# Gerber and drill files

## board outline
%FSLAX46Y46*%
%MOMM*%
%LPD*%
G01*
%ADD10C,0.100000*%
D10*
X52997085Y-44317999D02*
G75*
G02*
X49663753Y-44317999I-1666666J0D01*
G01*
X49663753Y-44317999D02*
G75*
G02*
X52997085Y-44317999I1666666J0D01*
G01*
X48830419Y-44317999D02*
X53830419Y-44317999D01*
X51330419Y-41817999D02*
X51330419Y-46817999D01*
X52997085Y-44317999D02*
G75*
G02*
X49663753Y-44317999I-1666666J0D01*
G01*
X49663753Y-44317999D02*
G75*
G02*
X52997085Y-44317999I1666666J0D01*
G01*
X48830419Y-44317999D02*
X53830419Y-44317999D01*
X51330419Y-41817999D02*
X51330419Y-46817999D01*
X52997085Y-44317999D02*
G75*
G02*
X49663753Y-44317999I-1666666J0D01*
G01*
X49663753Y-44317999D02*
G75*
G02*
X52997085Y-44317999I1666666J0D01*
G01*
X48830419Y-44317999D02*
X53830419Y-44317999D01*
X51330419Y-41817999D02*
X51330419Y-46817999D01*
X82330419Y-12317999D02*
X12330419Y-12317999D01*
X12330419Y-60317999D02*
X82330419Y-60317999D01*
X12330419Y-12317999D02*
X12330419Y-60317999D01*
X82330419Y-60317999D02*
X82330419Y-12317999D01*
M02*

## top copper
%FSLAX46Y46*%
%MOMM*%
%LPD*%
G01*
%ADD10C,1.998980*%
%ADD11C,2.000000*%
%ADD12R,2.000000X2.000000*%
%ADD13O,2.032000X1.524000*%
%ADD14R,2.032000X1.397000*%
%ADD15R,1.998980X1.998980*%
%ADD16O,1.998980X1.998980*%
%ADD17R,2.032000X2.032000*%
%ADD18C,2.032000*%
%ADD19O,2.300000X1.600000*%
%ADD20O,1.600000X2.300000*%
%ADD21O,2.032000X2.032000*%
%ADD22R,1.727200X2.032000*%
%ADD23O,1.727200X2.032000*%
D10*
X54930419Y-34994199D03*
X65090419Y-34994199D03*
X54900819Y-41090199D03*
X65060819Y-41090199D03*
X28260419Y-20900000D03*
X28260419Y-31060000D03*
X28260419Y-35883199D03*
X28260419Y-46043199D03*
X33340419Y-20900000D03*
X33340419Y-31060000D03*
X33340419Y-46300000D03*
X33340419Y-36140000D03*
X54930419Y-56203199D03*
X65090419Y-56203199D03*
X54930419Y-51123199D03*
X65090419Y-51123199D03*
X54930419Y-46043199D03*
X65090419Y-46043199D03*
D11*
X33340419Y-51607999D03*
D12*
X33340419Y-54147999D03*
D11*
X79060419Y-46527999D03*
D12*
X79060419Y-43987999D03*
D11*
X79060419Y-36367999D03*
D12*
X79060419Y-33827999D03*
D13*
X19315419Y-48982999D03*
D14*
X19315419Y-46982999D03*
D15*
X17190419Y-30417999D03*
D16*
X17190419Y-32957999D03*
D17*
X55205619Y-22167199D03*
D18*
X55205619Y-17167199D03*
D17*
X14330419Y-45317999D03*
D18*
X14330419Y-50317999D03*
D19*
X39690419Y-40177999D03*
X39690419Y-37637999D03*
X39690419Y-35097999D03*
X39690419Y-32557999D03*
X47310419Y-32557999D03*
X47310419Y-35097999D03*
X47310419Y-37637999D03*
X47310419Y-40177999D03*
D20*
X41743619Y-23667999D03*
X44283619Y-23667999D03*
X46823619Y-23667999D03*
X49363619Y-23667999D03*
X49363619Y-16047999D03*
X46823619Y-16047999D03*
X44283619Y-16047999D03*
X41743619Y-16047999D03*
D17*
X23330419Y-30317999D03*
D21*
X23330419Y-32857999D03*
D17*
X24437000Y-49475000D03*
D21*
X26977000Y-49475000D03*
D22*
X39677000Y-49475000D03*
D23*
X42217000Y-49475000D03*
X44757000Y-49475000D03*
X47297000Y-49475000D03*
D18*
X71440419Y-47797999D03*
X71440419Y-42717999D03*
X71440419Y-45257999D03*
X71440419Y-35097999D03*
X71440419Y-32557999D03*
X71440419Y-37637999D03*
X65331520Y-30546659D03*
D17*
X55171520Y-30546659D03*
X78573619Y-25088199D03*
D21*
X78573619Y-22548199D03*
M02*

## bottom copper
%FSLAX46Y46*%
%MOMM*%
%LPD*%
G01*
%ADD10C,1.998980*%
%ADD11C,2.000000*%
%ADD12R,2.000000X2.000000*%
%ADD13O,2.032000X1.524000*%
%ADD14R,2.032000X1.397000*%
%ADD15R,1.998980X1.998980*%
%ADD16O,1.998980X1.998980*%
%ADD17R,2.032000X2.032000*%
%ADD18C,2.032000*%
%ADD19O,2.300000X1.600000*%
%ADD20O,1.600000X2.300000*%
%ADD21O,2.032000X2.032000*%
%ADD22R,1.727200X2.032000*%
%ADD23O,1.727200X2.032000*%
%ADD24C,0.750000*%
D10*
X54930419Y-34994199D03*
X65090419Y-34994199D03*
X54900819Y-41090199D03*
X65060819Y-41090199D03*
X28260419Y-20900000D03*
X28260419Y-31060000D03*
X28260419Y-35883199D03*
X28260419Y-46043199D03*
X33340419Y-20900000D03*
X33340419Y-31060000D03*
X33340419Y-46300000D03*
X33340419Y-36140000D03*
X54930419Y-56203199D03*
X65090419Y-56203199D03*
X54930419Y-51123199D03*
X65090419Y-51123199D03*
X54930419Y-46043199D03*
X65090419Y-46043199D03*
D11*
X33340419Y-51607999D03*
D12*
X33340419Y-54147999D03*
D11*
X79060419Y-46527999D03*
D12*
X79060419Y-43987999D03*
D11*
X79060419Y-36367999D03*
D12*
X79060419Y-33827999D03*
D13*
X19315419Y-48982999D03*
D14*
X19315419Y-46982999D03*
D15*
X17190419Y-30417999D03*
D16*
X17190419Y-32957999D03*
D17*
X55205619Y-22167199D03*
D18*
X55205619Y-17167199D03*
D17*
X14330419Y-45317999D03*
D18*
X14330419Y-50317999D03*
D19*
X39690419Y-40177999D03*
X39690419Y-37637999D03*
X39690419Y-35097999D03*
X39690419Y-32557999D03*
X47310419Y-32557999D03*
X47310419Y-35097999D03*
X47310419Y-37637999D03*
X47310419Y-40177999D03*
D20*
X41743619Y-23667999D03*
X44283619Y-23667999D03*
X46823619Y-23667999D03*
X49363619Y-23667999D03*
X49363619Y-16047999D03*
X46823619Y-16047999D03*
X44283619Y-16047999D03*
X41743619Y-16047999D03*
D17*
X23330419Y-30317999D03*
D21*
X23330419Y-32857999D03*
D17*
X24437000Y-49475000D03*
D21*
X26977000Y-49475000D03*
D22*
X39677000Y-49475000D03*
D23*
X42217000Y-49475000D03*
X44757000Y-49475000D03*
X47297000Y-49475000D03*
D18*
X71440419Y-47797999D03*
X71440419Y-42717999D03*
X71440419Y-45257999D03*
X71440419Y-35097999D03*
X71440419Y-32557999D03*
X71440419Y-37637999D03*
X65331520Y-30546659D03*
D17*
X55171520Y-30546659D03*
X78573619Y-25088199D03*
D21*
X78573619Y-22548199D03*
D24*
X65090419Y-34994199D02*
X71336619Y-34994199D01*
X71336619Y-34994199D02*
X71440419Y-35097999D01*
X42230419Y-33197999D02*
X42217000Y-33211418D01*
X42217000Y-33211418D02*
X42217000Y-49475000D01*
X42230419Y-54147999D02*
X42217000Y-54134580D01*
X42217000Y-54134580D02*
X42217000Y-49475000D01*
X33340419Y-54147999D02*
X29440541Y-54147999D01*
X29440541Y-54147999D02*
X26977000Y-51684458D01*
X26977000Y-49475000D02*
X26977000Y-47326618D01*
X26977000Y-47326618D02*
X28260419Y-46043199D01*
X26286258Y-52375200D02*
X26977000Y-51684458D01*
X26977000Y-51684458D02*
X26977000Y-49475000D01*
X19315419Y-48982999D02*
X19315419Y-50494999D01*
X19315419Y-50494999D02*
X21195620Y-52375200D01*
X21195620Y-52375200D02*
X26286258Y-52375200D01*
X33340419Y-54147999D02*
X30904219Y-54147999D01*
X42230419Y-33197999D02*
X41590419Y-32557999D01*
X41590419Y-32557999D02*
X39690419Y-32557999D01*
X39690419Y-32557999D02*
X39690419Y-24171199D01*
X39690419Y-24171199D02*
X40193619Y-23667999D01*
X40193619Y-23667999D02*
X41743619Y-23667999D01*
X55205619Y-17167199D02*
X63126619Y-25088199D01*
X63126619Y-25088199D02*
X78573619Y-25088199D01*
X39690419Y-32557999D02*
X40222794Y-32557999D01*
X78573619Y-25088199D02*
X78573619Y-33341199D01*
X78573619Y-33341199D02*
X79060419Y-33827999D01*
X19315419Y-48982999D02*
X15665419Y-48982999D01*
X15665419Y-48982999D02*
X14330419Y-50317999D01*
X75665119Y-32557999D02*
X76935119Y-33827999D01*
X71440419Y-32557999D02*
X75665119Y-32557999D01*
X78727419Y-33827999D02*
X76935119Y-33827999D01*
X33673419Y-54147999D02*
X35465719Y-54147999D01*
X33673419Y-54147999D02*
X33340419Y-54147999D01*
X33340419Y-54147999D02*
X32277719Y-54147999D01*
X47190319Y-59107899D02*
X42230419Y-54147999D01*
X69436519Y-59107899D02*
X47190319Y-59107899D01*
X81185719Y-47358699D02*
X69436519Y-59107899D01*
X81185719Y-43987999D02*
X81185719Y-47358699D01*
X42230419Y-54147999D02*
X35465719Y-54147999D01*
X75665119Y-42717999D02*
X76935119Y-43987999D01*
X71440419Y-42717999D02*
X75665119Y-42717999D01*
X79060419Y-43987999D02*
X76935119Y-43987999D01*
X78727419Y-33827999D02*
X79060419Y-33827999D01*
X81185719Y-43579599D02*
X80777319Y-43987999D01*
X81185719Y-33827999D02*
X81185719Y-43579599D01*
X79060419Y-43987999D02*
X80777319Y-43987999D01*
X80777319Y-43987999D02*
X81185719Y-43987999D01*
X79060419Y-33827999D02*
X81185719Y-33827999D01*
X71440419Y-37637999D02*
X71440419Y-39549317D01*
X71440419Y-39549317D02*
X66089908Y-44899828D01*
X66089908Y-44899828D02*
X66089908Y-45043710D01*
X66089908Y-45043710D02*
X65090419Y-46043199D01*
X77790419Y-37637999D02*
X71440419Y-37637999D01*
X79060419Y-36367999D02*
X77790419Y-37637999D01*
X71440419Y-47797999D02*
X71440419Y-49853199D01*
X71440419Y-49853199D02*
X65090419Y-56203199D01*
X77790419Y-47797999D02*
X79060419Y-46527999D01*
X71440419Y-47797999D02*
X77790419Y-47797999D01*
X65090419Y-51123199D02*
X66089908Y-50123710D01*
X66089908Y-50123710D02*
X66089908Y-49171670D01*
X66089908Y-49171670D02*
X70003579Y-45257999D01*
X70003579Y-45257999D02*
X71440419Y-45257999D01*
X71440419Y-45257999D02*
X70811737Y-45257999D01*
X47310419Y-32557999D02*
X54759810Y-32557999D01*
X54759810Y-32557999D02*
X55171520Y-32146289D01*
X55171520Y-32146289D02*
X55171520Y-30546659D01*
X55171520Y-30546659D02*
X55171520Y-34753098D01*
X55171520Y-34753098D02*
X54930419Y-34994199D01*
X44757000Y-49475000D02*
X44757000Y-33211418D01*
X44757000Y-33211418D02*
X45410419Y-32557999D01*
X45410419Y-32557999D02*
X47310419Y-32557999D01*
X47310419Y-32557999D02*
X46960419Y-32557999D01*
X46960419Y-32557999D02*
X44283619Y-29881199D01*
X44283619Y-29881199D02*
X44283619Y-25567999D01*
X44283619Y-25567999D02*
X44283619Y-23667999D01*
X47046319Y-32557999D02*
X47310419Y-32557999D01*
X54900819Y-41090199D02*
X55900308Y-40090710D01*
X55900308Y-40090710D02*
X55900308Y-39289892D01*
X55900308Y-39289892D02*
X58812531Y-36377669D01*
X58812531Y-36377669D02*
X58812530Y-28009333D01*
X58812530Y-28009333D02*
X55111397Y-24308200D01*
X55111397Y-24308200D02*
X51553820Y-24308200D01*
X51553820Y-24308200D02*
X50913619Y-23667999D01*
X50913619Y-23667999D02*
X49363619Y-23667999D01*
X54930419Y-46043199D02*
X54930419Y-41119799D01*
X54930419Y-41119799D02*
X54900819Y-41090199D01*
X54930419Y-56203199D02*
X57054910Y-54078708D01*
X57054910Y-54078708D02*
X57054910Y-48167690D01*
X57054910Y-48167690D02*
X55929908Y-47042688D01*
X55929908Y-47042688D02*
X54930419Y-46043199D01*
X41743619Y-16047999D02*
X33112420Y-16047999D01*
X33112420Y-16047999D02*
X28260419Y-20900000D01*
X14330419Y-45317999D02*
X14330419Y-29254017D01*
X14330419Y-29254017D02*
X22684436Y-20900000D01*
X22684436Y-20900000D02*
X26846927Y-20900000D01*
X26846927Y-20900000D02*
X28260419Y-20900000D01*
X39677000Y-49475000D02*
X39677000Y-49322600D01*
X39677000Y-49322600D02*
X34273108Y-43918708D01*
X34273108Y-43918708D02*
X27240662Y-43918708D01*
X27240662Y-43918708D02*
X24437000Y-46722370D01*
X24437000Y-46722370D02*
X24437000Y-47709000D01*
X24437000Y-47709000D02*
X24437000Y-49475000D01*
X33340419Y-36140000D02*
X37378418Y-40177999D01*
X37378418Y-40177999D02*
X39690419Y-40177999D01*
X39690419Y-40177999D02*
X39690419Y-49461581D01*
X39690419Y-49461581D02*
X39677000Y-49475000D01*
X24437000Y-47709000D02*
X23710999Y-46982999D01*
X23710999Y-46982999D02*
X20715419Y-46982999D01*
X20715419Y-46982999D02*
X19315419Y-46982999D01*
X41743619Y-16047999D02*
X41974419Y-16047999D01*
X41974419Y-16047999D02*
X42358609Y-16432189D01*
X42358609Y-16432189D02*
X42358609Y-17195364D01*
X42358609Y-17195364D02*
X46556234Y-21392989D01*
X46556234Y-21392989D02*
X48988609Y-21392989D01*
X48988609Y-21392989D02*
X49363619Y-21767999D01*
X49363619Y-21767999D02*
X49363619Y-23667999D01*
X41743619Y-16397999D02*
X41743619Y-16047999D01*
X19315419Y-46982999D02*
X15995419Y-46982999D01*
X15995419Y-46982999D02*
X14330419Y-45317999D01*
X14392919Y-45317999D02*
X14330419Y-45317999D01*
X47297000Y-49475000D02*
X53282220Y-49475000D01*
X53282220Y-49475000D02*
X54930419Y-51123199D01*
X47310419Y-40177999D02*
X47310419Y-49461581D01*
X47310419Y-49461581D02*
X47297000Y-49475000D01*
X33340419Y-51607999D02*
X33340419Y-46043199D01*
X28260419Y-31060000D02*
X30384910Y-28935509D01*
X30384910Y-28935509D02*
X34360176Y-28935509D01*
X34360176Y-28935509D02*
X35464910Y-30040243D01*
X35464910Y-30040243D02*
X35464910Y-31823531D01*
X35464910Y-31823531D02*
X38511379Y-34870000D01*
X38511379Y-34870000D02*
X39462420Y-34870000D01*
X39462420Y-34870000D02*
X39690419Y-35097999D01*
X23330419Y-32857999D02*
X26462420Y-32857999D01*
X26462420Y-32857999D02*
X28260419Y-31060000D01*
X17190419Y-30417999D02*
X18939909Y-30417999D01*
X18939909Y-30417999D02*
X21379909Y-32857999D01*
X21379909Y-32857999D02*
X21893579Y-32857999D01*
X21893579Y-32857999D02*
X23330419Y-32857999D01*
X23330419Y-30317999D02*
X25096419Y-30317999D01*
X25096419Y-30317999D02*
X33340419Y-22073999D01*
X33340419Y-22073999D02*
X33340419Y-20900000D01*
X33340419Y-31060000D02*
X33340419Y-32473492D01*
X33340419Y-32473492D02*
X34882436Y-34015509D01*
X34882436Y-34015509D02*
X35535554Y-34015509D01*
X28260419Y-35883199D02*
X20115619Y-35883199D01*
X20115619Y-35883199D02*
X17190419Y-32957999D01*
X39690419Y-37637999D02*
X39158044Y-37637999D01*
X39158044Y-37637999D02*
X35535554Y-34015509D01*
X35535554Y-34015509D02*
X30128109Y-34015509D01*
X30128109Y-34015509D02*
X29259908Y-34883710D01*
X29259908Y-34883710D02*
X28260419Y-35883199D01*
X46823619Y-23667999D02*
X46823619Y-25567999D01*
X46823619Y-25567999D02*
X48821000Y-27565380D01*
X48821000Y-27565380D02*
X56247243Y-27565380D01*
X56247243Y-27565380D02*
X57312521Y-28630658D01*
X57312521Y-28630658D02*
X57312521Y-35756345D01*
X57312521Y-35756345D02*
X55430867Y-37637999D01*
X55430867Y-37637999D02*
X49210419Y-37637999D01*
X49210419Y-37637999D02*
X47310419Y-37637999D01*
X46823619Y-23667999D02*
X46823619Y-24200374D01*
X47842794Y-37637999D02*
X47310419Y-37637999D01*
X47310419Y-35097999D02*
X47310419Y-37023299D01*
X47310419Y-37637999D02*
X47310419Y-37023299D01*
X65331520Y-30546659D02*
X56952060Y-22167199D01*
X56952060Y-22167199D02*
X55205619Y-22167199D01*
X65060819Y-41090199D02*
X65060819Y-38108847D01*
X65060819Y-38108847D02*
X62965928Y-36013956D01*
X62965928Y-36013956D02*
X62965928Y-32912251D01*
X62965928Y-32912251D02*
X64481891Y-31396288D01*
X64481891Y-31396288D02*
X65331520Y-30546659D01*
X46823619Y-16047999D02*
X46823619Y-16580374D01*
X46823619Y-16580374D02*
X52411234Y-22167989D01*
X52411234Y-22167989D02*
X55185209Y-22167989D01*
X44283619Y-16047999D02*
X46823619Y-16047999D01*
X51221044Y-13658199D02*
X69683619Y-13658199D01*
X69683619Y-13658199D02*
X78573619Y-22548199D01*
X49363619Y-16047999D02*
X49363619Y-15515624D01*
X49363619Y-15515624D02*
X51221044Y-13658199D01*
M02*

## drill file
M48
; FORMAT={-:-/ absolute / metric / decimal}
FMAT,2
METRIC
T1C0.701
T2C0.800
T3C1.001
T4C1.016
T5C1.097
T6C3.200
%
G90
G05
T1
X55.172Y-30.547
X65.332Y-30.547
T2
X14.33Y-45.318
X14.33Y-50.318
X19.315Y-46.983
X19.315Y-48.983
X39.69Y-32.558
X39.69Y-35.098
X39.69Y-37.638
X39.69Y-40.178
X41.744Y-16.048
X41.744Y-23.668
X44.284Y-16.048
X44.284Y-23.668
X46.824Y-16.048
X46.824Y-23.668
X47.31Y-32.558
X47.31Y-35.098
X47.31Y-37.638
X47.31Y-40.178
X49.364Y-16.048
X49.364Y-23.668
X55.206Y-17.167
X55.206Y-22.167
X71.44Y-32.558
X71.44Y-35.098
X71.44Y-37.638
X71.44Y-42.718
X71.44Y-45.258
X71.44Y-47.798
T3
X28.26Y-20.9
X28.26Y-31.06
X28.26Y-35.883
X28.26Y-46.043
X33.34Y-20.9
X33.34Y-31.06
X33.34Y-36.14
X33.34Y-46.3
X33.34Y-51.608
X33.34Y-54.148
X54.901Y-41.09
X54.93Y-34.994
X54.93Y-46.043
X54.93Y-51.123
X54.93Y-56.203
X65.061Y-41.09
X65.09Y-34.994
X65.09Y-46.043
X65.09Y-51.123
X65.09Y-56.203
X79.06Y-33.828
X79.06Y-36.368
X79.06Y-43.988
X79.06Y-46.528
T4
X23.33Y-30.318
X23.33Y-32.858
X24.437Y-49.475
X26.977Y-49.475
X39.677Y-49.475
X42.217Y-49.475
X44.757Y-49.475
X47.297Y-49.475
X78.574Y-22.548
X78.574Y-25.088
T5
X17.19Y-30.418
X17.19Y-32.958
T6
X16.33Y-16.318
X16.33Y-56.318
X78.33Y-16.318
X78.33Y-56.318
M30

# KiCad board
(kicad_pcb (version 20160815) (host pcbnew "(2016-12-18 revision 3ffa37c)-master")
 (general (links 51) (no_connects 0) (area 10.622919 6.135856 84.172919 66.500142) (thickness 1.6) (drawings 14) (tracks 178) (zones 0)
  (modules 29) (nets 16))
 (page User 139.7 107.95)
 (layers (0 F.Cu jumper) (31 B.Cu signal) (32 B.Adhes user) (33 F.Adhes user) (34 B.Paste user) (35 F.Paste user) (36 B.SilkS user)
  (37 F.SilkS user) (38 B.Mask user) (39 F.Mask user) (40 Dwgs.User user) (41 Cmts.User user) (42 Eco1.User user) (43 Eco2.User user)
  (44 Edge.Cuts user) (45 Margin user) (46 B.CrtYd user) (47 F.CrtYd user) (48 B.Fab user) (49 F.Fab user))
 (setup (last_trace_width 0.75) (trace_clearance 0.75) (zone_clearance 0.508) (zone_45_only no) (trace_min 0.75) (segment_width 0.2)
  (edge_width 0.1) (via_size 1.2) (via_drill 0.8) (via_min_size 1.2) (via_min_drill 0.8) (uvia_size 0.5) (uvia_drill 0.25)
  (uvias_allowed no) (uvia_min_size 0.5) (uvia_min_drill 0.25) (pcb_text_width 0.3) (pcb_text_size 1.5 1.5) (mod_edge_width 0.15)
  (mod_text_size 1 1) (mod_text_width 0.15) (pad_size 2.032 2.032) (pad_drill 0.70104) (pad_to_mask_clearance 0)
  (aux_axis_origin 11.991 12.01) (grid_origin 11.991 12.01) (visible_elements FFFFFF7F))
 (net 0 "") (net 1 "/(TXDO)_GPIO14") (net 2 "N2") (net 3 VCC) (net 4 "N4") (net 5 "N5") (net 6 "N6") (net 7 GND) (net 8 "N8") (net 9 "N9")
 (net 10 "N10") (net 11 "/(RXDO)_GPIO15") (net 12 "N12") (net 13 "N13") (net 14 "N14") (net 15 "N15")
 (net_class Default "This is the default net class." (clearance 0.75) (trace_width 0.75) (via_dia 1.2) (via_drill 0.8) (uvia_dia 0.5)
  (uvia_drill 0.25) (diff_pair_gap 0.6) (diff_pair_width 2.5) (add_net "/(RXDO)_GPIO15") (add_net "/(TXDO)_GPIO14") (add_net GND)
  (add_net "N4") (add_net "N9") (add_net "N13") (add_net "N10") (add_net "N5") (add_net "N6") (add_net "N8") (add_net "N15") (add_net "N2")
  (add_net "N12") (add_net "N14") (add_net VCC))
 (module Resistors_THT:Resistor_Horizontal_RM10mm (layer F.Cu) (at 65.090419 34.994199 180)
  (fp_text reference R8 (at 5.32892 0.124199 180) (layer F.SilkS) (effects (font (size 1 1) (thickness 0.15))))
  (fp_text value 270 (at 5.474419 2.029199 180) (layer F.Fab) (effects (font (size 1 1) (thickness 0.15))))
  (pad 2 thru_hole circle (at 10.16 0 180) (size 1.99898 1.99898) (drill 1.00076) (layers *.Cu *.SilkS *.Mask) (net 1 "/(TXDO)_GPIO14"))
  (pad 1 thru_hole circle (at 0 0 180) (size 1.99898 1.99898) (drill 1.00076) (layers *.Cu *.SilkS *.Mask) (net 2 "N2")))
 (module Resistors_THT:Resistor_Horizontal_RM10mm (layer F.Cu) (at 65.060819 41.090199 180)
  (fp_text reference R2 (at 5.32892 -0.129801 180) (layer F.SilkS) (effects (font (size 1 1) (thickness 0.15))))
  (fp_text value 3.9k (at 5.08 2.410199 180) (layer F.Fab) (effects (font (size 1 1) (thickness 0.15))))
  (pad 2 thru_hole circle (at 10.16 0 180) (size 1.99898 1.99898) (drill 1.00076) (layers *.Cu *.SilkS *.Mask) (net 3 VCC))
  (pad 1 thru_hole circle (at 0 0 180) (size 1.99898 1.99898) (drill 1.00076) (layers *.Cu *.SilkS *.Mask) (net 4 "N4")))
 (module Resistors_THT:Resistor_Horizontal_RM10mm (layer F.Cu) (at 28.260419 31.06 90)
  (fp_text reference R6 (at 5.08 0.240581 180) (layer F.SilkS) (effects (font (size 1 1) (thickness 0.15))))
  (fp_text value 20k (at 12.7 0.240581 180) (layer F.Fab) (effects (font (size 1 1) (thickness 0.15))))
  (pad 2 thru_hole circle (at 10.16 0 90) (size 1.99898 1.99898) (drill 1.00076) (layers *.Cu *.SilkS *.Mask) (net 3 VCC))
  (pad 1 thru_hole circle (at 0 0 90) (size 1.99898 1.99898) (drill 1.00076) (layers *.Cu *.SilkS *.Mask) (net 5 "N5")))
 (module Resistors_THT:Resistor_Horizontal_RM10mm (layer F.Cu) (at 28.260419 46.043199 90)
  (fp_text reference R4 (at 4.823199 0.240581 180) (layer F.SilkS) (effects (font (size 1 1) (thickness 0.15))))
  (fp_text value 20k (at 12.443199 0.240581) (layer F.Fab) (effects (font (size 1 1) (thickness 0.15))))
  (pad 2 thru_hole circle (at 10.16 0 90) (size 1.99898 1.99898) (drill 1.00076) (layers *.Cu *.SilkS *.Mask) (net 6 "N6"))
  (pad 1 thru_hole circle (at 0 0 90) (size 1.99898 1.99898) (drill 1.00076) (layers *.Cu *.SilkS *.Mask) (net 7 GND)))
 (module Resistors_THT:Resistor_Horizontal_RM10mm (layer F.Cu) (at 33.340419 31.06 90)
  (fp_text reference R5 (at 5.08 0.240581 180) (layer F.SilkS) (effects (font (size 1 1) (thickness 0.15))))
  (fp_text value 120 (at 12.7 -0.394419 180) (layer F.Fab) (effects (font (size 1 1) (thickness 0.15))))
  (pad 2 thru_hole circle (at 10.16 0 90) (size 1.99898 1.99898) (drill 1.00076) (layers *.Cu *.SilkS *.Mask) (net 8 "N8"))
  (pad 1 thru_hole circle (at 0 0 90) (size 1.99898 1.99898) (drill 1.00076) (layers *.Cu *.SilkS *.Mask) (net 6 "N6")))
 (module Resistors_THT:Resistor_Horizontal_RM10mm (layer F.Cu) (at 33.340419 36.14 270)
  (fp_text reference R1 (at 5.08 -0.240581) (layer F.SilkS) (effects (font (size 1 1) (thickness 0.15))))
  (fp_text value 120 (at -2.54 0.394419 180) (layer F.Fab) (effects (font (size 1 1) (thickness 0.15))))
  (pad 2 thru_hole circle (at 10.16 0 270) (size 1.99898 1.99898) (drill 1.00076) (layers *.Cu *.SilkS *.Mask) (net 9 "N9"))
  (pad 1 thru_hole circle (at 0 0 270) (size 1.99898 1.99898) (drill 1.00076) (layers *.Cu *.SilkS *.Mask) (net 3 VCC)))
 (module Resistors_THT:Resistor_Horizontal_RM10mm (layer F.Cu) (at 65.090419 56.203199 180)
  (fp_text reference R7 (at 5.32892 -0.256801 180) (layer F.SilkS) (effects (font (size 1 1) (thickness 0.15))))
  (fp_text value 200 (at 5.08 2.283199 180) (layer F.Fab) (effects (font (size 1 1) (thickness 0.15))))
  (pad 2 thru_hole circle (at 10.16 0 180) (size 1.99898 1.99898) (drill 1.00076) (layers *.Cu *.SilkS *.Mask) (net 3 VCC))
  (pad 1 thru_hole circle (at 0 0 180) (size 1.99898 1.99898) (drill 1.00076) (layers *.Cu *.SilkS *.Mask) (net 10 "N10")))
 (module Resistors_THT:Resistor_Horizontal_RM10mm (layer F.Cu) (at 65.090419 51.123199 180)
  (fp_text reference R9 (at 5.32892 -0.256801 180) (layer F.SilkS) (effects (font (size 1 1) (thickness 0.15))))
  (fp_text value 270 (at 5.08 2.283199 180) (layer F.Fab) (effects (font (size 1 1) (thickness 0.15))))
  (pad 2 thru_hole circle (at 10.16 0 180) (size 1.99898 1.99898) (drill 1.00076) (layers *.Cu *.SilkS *.Mask) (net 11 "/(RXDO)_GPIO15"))
  (pad 1 thru_hole circle (at 0 0 180) (size 1.99898 1.99898) (drill 1.00076) (layers *.Cu *.SilkS *.Mask) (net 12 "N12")))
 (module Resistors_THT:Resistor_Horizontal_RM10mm (layer F.Cu) (at 65.090419 46.043199 180)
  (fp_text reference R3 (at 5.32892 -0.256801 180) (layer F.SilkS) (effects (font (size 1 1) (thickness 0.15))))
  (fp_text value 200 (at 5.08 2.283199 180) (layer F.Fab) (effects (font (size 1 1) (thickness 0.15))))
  (pad 2 thru_hole circle (at 10.16 0 180) (size 1.99898 1.99898) (drill 1.00076) (layers *.Cu *.SilkS *.Mask) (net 3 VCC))
  (pad 1 thru_hole circle (at 0 0 180) (size 1.99898 1.99898) (drill 1.00076) (layers *.Cu *.SilkS *.Mask) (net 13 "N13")))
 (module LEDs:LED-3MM (layer F.Cu) (at 33.340419 54.147999 90)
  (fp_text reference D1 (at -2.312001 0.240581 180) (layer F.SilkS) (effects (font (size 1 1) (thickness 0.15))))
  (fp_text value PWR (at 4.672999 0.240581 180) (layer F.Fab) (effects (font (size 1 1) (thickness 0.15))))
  (pad 2 thru_hole circle (at 2.54 0 90) (size 2 2) (drill 1.00076) (layers *.Cu *.Mask) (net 9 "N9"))
  (pad 1 thru_hole rect (at 0 0 180) (size 2 2) (drill 1.00076) (layers *.Cu *.Mask) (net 7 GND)))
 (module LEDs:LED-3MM (layer F.Cu) (at 79.060419 43.987999 270)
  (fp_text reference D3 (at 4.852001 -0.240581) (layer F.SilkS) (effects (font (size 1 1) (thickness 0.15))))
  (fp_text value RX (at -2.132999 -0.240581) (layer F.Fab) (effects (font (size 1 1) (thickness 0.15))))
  (pad 2 thru_hole circle (at 2.54 0 270) (size 2 2) (drill 1.00076) (layers *.Cu *.Mask) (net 10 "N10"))
  (pad 1 thru_hole rect (at 0 0) (size 2 2) (drill 1.00076) (layers *.Cu *.Mask) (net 7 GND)))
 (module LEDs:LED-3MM (layer F.Cu) (at 79.060419 33.827999 270)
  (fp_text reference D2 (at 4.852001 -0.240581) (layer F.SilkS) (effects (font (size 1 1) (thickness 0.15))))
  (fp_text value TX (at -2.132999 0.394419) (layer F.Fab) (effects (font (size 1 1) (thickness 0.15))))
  (pad 2 thru_hole circle (at 2.54 0 270) (size 2 2) (drill 1.00076) (layers *.Cu *.Mask) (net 13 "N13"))
  (pad 1 thru_hole rect (at 0 0) (size 2 2) (drill 1.00076) (layers *.Cu *.Mask) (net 7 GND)))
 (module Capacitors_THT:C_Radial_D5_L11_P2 (layer F.Cu) (at 19.315419 46.982999 270)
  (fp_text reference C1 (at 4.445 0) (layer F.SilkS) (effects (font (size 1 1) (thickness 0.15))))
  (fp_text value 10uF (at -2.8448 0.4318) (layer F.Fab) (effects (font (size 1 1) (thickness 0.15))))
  (pad 2 thru_hole oval (at 2 0 270) (size 1.524 2.032) (drill 0.8) (layers *.Cu *.Mask) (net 7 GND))
  (pad 1 thru_hole rect (at 0 0 270) (size 1.397 2.032) (drill 0.8) (layers *.Cu *.Mask) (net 3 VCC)))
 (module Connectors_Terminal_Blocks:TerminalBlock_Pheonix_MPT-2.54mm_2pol (layer F.Cu) (at 17.190419 30.417999 270)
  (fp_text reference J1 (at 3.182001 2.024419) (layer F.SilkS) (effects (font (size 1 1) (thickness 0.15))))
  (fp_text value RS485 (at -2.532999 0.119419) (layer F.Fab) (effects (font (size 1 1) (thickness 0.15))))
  (pad 1 thru_hole rect (at 0 0 270) (size 1.99898 1.99898) (drill 1.09728) (layers *.Cu *.Mask) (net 5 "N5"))
  (pad 2 thru_hole oval (at 2.54 0 270) (size 1.99898 1.99898) (drill 1.09728) (layers *.Cu *.Mask) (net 6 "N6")))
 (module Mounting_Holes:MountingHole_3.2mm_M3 (layer F.Cu) (at 78.330419 56.317999 90)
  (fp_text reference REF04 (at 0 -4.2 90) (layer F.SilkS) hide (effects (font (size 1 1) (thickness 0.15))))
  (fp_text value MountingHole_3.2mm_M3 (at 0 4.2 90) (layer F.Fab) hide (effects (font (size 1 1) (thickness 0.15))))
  (pad "" np_thru_hole circle (at 0 0 90) (size 3.2 3.2) (drill 3.2) (layers *.Cu *.Mask F.SilkS)))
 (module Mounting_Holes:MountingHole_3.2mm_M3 (layer F.Cu) (at 78.330419 16.317999 90)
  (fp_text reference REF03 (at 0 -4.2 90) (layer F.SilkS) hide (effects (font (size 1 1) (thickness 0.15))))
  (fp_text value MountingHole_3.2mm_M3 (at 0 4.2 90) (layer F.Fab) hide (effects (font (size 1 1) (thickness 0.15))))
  (pad "" np_thru_hole circle (at 0 0 90) (size 3.2 3.2) (drill 3.2) (layers *.Cu *.Mask F.SilkS)))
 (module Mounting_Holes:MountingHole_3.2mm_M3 (layer F.Cu) (at 16.330419 16.317999 90)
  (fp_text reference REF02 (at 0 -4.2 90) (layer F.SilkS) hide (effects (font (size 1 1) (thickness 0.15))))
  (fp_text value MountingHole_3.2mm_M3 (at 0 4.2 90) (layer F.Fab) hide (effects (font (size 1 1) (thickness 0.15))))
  (pad "" np_thru_hole circle (at 0 0 90) (size 3.2 3.2) (drill 3.2) (layers *.Cu *.Mask F.SilkS)))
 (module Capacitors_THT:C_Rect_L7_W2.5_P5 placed (layer F.Cu) (at 55.205619 22.167199 90)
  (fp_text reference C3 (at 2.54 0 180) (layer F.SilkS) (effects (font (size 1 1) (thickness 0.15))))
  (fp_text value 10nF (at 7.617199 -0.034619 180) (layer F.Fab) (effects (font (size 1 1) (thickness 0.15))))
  (pad 1 thru_hole rect (at 0 0 90) (size 2.032 2.032) (drill 0.8) (layers *.Cu *.Mask) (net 4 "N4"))
  (pad 2 thru_hole circle (at 5 0 90) (size 2.032 2.032) (drill 0.8) (layers *.Cu *.Mask) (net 7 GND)))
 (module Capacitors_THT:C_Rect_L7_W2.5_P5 (layer F.Cu) (at 14.330419 45.317999 270)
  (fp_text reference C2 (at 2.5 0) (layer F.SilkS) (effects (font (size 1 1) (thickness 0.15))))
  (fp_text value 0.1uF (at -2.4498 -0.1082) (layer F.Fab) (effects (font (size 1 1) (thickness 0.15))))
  (pad 1 thru_hole rect (at 0 0 270) (size 2.032 2.032) (drill 0.8) (layers *.Cu *.Mask) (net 3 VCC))
  (pad 2 thru_hole circle (at 5 0 270) (size 2.032 2.032) (drill 0.8) (layers *.Cu *.Mask) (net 7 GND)))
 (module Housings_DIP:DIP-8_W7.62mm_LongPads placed (layer F.Cu) (at 47.310419 40.177999 180)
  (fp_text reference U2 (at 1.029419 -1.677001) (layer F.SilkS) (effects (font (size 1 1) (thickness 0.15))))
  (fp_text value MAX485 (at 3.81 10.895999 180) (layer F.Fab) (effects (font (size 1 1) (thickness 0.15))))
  (pad 8 thru_hole oval (at 7.62 0 180) (size 2.3 1.6) (drill 0.8) (layers *.Cu *.Mask) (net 3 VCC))
  (pad 7 thru_hole oval (at 7.62 2.54 180) (size 2.3 1.6) (drill 0.8) (layers *.Cu *.Mask) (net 6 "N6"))
  (pad 6 thru_hole oval (at 7.62 5.08 180) (size 2.3 1.6) (drill 0.8) (layers *.Cu *.Mask) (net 5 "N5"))
  (pad 5 thru_hole oval (at 7.62 7.62 180) (size 2.3 1.6) (drill 0.8) (layers *.Cu *.Mask) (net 7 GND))
  (pad 4 thru_hole oval (at 0 7.62 180) (size 2.3 1.6) (drill 0.8) (layers *.Cu *.Mask) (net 1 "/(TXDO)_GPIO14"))
  (pad 3 thru_hole oval (at 0 5.08 180) (size 2.3 1.6) (drill 0.8) (layers *.Cu *.Mask) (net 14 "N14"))
  (pad 2 thru_hole oval (at 0 2.54 180) (size 2.3 1.6) (drill 0.8) (layers *.Cu *.Mask) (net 14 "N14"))
  (pad 1 thru_hole oval (at 0 0 180) (size 2.3 1.6) (drill 0.8) (layers *.Cu *.Mask) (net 11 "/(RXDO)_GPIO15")))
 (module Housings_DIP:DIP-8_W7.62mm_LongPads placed (layer F.Cu) (at 41.743619 23.667999 90)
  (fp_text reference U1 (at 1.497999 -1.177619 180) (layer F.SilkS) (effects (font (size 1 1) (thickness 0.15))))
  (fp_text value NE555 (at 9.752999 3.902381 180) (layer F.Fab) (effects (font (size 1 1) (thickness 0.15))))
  (pad 1 thru_hole oval (at 0 0 90) (size 2.3 1.6) (drill 0.8) (layers *.Cu *.Mask) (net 7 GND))
  (pad 2 thru_hole oval (at 0 2.54 90) (size 2.3 1.6) (drill 0.8) (layers *.Cu *.Mask) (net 1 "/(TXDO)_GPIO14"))
  (pad 3 thru_hole oval (at 0 5.08 90) (size 2.3 1.6) (drill 0.8) (layers *.Cu *.Mask) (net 14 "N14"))
  (pad 4 thru_hole oval (at 0 7.62 90) (size 2.3 1.6) (drill 0.8) (layers *.Cu *.Mask) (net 3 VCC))
  (pad 5 thru_hole oval (at 7.62 7.62 90) (size 2.3 1.6) (drill 0.8) (layers *.Cu *.Mask) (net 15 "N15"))
  (pad 6 thru_hole oval (at 7.62 5.08 90) (size 2.3 1.6) (drill 0.8) (layers *.Cu *.Mask) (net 4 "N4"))
  (pad 7 thru_hole oval (at 7.62 2.54 90) (size 2.3 1.6) (drill 0.8) (layers *.Cu *.Mask) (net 4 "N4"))
  (pad 8 thru_hole oval (at 7.62 0 90) (size 2.3 1.6) (drill 0.8) (layers *.Cu *.Mask) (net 3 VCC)))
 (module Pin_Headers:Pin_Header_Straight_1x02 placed (layer F.Cu) (at 23.330419 30.317999)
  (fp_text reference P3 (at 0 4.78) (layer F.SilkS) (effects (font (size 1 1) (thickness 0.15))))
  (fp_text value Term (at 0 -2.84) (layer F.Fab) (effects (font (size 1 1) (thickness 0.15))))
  (pad 1 thru_hole rect (at 0 0) (size 2.032 2.032) (drill 1.016) (layers *.Cu *.Mask) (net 8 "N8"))
  (pad 2 thru_hole oval (at 0 2.54) (size 2.032 2.032) (drill 1.016) (layers *.Cu *.Mask) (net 5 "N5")))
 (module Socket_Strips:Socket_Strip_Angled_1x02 (layer F.Cu) (at 24.437 49.475)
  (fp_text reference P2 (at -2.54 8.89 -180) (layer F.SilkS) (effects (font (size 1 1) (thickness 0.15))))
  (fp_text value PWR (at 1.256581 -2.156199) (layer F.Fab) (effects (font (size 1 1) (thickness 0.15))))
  (pad 1 thru_hole rect (at 0 0) (size 2.032 2.032) (drill 1.016) (layers *.Cu *.Mask) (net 3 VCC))
  (pad 2 thru_hole oval (at 2.54 0) (size 2.032 2.032) (drill 1.016) (layers *.Cu *.Mask) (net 7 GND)))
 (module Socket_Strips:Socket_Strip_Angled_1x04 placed (layer F.Cu) (at 39.677 49.475)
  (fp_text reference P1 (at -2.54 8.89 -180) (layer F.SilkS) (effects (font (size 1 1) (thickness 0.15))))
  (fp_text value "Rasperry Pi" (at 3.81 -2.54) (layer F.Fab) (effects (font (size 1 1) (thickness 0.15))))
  (pad 1 thru_hole rect (at 0 0) (size 1.7272 2.032) (drill 1.016) (layers *.Cu *.Mask) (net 3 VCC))
  (pad 2 thru_hole oval (at 2.54 0) (size 1.7272 2.032) (drill 1.016) (layers *.Cu *.Mask) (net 7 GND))
  (pad 3 thru_hole oval (at 5.08 0) (size 1.7272 2.032) (drill 1.016) (layers *.Cu *.Mask) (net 1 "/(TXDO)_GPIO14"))
  (pad 4 thru_hole oval (at 7.62 0) (size 1.7272 2.032) (drill 1.016) (layers *.Cu *.Mask) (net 11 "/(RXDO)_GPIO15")))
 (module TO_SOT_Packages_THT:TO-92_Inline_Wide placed (layer F.Cu) (at 71.440419 47.797999 90)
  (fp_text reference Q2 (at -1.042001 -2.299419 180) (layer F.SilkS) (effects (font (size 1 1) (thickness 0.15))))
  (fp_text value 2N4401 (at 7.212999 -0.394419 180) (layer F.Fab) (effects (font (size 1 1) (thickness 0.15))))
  (pad 1 thru_hole circle (at 0 0 180) (size 2.032 2.032) (drill 0.8) (layers *.Cu *.Mask) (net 10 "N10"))
  (pad 3 thru_hole circle (at 5.08 0 180) (size 2.032 2.032) (drill 0.8) (layers *.Cu *.Mask) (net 7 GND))
  (pad 2 thru_hole circle (at 2.54 0 180) (size 2.032 2.032) (drill 0.8) (layers *.Cu *.Mask) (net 12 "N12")))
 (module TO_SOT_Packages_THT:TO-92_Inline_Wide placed (layer F.Cu) (at 71.440419 37.637999 90)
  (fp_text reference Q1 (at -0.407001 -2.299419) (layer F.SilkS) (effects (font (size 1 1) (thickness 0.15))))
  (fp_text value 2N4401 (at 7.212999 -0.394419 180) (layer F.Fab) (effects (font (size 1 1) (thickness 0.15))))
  (pad 2 thru_hole circle (at 2.54 0 180) (size 2.032 2.032) (drill 0.8) (layers *.Cu *.Mask) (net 2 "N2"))
  (pad 3 thru_hole circle (at 5.08 0 180) (size 2.032 2.032) (drill 0.8) (layers *.Cu *.Mask) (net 7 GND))
  (pad 1 thru_hole circle (at 0 0 180) (size 2.032 2.032) (drill 0.8) (layers *.Cu *.Mask) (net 13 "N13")))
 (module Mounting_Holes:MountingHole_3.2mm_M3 (layer F.Cu) (at 16.330419 56.317999 90)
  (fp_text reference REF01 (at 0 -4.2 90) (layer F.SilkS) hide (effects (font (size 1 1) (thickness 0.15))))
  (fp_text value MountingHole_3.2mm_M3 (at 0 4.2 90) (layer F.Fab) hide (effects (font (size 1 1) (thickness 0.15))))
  (pad "" np_thru_hole circle (at 0 0 90) (size 3.2 3.2) (drill 3.2) (layers *.Cu *.Mask F.SilkS)))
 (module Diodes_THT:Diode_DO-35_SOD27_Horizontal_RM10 (layer F.Cu) (at 55.171 30.549199)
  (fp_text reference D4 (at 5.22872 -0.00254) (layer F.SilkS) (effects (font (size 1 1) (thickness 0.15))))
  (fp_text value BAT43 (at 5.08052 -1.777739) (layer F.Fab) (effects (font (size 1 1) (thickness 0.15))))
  (pad 2 thru_hole circle (at 10.16052 -0.00254 180) (size 2.032 2.032) (drill 0.70104) (layers *.Cu *.Mask) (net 4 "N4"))
  (pad 1 thru_hole rect (at 0.00052 -0.00254 180) (size 2.032 2.032) (drill 0.70104) (layers *.Cu *.Mask) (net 1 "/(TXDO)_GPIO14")))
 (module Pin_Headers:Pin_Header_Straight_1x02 (layer F.Cu) (at 78.573619 25.088199 180)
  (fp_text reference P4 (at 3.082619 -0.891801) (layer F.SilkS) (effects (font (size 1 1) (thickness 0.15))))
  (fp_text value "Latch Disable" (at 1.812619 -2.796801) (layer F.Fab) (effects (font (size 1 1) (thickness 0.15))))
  (pad 1 thru_hole rect (at 0 0 180) (size 2.032 2.032) (drill 1.016) (layers *.Cu *.Mask) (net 7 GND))
  (pad 2 thru_hole oval (at 0 2.54 180) (size 2.032 2.032) (drill 1.016) (layers *.Cu *.Mask) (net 15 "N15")))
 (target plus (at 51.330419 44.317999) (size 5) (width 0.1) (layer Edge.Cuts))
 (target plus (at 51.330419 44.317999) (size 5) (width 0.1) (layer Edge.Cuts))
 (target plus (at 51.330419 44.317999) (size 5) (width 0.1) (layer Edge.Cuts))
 (gr_line (start 82.330419 12.317999) (end 12.330419 12.317999) (angle 90) (layer Edge.Cuts) (width 0.1))
 (gr_line (start 12.330419 60.317999) (end 82.330419 60.317999) (angle 90) (layer Edge.Cuts) (width 0.1))
 (gr_line (start 12.330419 12.317999) (end 12.330419 60.317999) (angle 90) (layer Edge.Cuts) (width 0.1))
 (gr_line (start 82.330419 60.317999) (end 82.330419 12.317999) (angle 90) (layer Edge.Cuts) (width 0.1))
 (segment (start 65.090419 34.994199) (end 71.336619 34.994199) (width 0.75) (layer B.Cu) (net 2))
 (segment (start 71.336619 34.994199) (end 71.440419 35.097999) (width 0.75) (layer B.Cu) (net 2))
 (segment (start 42.230419 33.197999) (end 42.217 33.211418) (width 0.75) (layer B.Cu) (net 7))
 (segment (start 42.217 33.211418) (end 42.217 49.475) (width 0.75) (layer B.Cu) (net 7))
 (segment (start 42.230419 54.147999) (end 42.217 54.13458) (width 0.75) (layer B.Cu) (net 7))
 (segment (start 42.217 54.13458) (end 42.217 49.475) (width 0.75) (layer B.Cu) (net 7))
 (segment (start 33.340419 54.147999) (end 29.440541 54.147999) (width 0.75) (layer B.Cu) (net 7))
 (segment (start 29.440541 54.147999) (end 26.977 51.684458) (width 0.75) (layer B.Cu) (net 7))
 (segment (start 26.977 49.475) (end 26.977 47.326618) (width 0.75) (layer B.Cu) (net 7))
 (segment (start 26.977 47.326618) (end 28.260419 46.043199) (width 0.75) (layer B.Cu) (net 7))
 (segment (start 26.286258 52.3752) (end 26.977 51.684458) (width 0.75) (layer B.Cu) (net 7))
 (segment (start 26.977 51.684458) (end 26.977 49.475) (width 0.75) (layer B.Cu) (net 7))
 (segment (start 19.315419 48.982999) (end 19.315419 50.494999) (width 0.75) (layer B.Cu) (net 7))
 (segment (start 19.315419 50.494999) (end 21.19562 52.3752) (width 0.75) (layer B.Cu) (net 7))
 (segment (start 21.19562 52.3752) (end 26.286258 52.3752) (width 0.75) (layer B.Cu) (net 7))
 (segment (start 33.340419 54.147999) (end 30.904219 54.147999) (width 0.75) (layer B.Cu) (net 7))
 (segment (start 42.230419 33.197999) (end 41.590419 32.557999) (width 0.75) (layer B.Cu) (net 7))
 (segment (start 41.590419 32.557999) (end 39.690419 32.557999) (width 0.75) (layer B.Cu) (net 7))
 (segment (start 39.690419 32.557999) (end 39.690419 24.171199) (width 0.75) (layer B.Cu) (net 7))
 (segment (start 39.690419 24.171199) (end 40.193619 23.667999) (width 0.75) (layer B.Cu) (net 7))
 (segment (start 40.193619 23.667999) (end 41.743619 23.667999) (width 0.75) (layer B.Cu) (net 7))
 (segment (start 55.205619 17.167199) (end 63.126619 25.088199) (width 0.75) (layer B.Cu) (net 7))
 (segment (start 63.126619 25.088199) (end 78.573619 25.088199) (width 0.75) (layer B.Cu) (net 7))
 (segment (start 39.690419 32.557999) (end 40.222794 32.557999) (width 0.75) (layer B.Cu) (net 7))
 (segment (start 78.573619 25.088199) (end 78.573619 33.341199) (width 0.75) (layer B.Cu) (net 7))
 (segment (start 78.573619 33.341199) (end 79.060419 33.827999) (width 0.75) (layer B.Cu) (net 7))
 (segment (start 19.315419 48.982999) (end 15.665419 48.982999) (width 0.75) (layer B.Cu) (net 7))
 (segment (start 15.665419 48.982999) (end 14.330419 50.317999) (width 0.75) (layer B.Cu) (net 7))
 (segment (start 75.665119 32.557999) (end 76.935119 33.827999) (width 0.75) (layer B.Cu) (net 7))
 (segment (start 71.440419 32.557999) (end 75.665119 32.557999) (width 0.75) (layer B.Cu) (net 7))
 (segment (start 78.727419 33.827999) (end 76.935119 33.827999) (width 0.75) (layer B.Cu) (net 7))
 (segment (start 33.673419 54.147999) (end 35.465719 54.147999) (width 0.75) (layer B.Cu) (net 7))
 (segment (start 33.673419 54.147999) (end 33.340419 54.147999) (width 0.75) (layer B.Cu) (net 7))
 (segment (start 33.340419 54.147999) (end 32.277719 54.147999) (width 0.75) (layer B.Cu) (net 7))
 (segment (start 47.190319 59.107899) (end 42.230419 54.147999) (width 0.75) (layer B.Cu) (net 7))
 (segment (start 69.436519 59.107899) (end 47.190319 59.107899) (width 0.75) (layer B.Cu) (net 7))
 (segment (start 81.185719 47.358699) (end 69.436519 59.107899) (width 0.75) (layer B.Cu) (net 7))
 (segment (start 81.185719 43.987999) (end 81.185719 47.358699) (width 0.75) (layer B.Cu) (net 7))
 (segment (start 42.230419 54.147999) (end 35.465719 54.147999) (width 0.75) (layer B.Cu) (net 7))
 (segment (start 75.665119 42.717999) (end 76.935119 43.987999) (width 0.75) (layer B.Cu) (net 7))
 (segment (start 71.440419 42.717999) (end 75.665119 42.717999) (width 0.75) (layer B.Cu) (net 7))
 (segment (start 79.060419 43.987999) (end 76.935119 43.987999) (width 0.75) (layer B.Cu) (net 7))
 (segment (start 78.727419 33.827999) (end 79.060419 33.827999) (width 0.75) (layer B.Cu) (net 7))
 (segment (start 81.185719 43.579599) (end 80.777319 43.987999) (width 0.75) (layer B.Cu) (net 7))
 (segment (start 81.185719 33.827999) (end 81.185719 43.579599) (width 0.75) (layer B.Cu) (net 7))
 (segment (start 79.060419 43.987999) (end 80.777319 43.987999) (width 0.75) (layer B.Cu) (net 7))
 (segment (start 80.777319 43.987999) (end 81.185719 43.987999) (width 0.75) (layer B.Cu) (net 7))
 (segment (start 79.060419 33.827999) (end 81.185719 33.827999) (width 0.75) (layer B.Cu) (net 7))
 (segment (start 71.440419 37.637999) (end 71.440419 39.549317) (width 0.75) (layer B.Cu) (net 13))
 (segment (start 71.440419 39.549317) (end 66.089908 44.899828) (width 0.75) (layer B.Cu) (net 13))
 (segment (start 66.089908 44.899828) (end 66.089908 45.04371) (width 0.75) (layer B.Cu) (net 13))
 (segment (start 66.089908 45.04371) (end 65.090419 46.043199) (width 0.75) (layer B.Cu) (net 13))
 (segment (start 77.790419 37.637999) (end 71.440419 37.637999) (width 0.75) (layer B.Cu) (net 13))
 (segment (start 79.060419 36.367999) (end 77.790419 37.637999) (width 0.75) (layer B.Cu) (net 13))
 (segment (start 71.440419 47.797999) (end 71.440419 49.853199) (width 0.75) (layer B.Cu) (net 10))
 (segment (start 71.440419 49.853199) (end 65.090419 56.203199) (width 0.75) (layer B.Cu) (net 10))
 (segment (start 77.790419 47.797999) (end 79.060419 46.527999) (width 0.75) (layer B.Cu) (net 10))
 (segment (start 71.440419 47.797999) (end 77.790419 47.797999) (width 0.75) (layer B.Cu) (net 10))
 (segment (start 65.090419 51.123199) (end 66.089908 50.12371) (width 0.75) (layer B.Cu) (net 12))
 (segment (start 66.089908 50.12371) (end 66.089908 49.17167) (width 0.75) (layer B.Cu) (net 12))
 (segment (start 66.089908 49.17167) (end 70.003579 45.257999) (width 0.75) (layer B.Cu) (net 12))
 (segment (start 70.003579 45.257999) (end 71.440419 45.257999) (width 0.75) (layer B.Cu) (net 12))
 (segment (start 71.440419 45.257999) (end 70.811737 45.257999) (width 0.75) (layer B.Cu) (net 12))
 (segment (start 47.310419 32.557999) (end 54.75981 32.557999) (width 0.75) (layer B.Cu) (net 1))
 (segment (start 54.75981 32.557999) (end 55.17152 32.146289) (width 0.75) (layer B.Cu) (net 1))
 (segment (start 55.17152 32.146289) (end 55.17152 30.546659) (width 0.75) (layer B.Cu) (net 1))
 (segment (start 55.17152 30.546659) (end 55.17152 34.753098) (width 0.75) (layer B.Cu) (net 1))
 (segment (start 55.17152 34.753098) (end 54.930419 34.994199) (width 0.75) (layer B.Cu) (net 1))
 (segment (start 44.757 49.475) (end 44.757 33.211418) (width 0.75) (layer B.Cu) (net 1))
 (segment (start 44.757 33.211418) (end 45.410419 32.557999) (width 0.75) (layer B.Cu) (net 1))
 (segment (start 45.410419 32.557999) (end 47.310419 32.557999) (width 0.75) (layer B.Cu) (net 1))
 (segment (start 47.310419 32.557999) (end 46.960419 32.557999) (width 0.75) (layer B.Cu) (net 1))
 (segment (start 46.960419 32.557999) (end 44.283619 29.881199) (width 0.75) (layer B.Cu) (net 1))
 (segment (start 44.283619 29.881199) (end 44.283619 25.567999) (width 0.75) (layer B.Cu) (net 1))
 (segment (start 44.283619 25.567999) (end 44.283619 23.667999) (width 0.75) (layer B.Cu) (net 1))
 (segment (start 47.046319 32.557999) (end 47.310419 32.557999) (width 0.75) (layer B.Cu) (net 1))
 (segment (start 54.900819 41.090199) (end 55.900308 40.09071) (width 0.75) (layer B.Cu) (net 3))
 (segment (start 55.900308 40.09071) (end 55.900308 39.289892) (width 0.75) (layer B.Cu) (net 3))
 (segment (start 55.900308 39.289892) (end 58.812531 36.377669) (width 0.75) (layer B.Cu) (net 3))
 (segment (start 58.812531 36.377669) (end 58.81253 28.009333) (width 0.75) (layer B.Cu) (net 3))
 (segment (start 58.81253 28.009333) (end 55.111397 24.3082) (width 0.75) (layer B.Cu) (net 3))
 (segment (start 55.111397 24.3082) (end 51.55382 24.3082) (width 0.75) (layer B.Cu) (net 3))
 (segment (start 51.55382 24.3082) (end 50.913619 23.667999) (width 0.75) (layer B.Cu) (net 3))
 (segment (start 50.913619 23.667999) (end 49.363619 23.667999) (width 0.75) (layer B.Cu) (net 3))
 (segment (start 54.930419 46.043199) (end 54.930419 41.119799) (width 0.75) (layer B.Cu) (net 3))
 (segment (start 54.930419 41.119799) (end 54.900819 41.090199) (width 0.75) (layer B.Cu) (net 3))
 (segment (start 54.930419 56.203199) (end 57.05491 54.078708) (width 0.75) (layer B.Cu) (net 3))
 (segment (start 57.05491 54.078708) (end 57.05491 48.16769) (width 0.75) (layer B.Cu) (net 3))
 (segment (start 57.05491 48.16769) (end 55.929908 47.042688) (width 0.75) (layer B.Cu) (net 3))
 (segment (start 55.929908 47.042688) (end 54.930419 46.043199) (width 0.75) (layer B.Cu) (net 3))
 (segment (start 41.743619 16.047999) (end 33.11242 16.047999) (width 0.75) (layer B.Cu) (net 3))
 (segment (start 33.11242 16.047999) (end 28.260419 20.9) (width 0.75) (layer B.Cu) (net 3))
 (segment (start 14.330419 45.317999) (end 14.330419 29.254017) (width 0.75) (layer B.Cu) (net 3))
 (segment (start 14.330419 29.254017) (end 22.684436 20.9) (width 0.75) (layer B.Cu) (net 3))
 (segment (start 22.684436 20.9) (end 26.846927 20.9) (width 0.75) (layer B.Cu) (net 3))
 (segment (start 26.846927 20.9) (end 28.260419 20.9) (width 0.75) (layer B.Cu) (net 3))
 (segment (start 39.677 49.475) (end 39.677 49.3226) (width 0.75) (layer B.Cu) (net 3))
 (segment (start 39.677 49.3226) (end 34.273108 43.918708) (width 0.75) (layer B.Cu) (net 3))
 (segment (start 34.273108 43.918708) (end 27.240662 43.918708) (width 0.75) (layer B.Cu) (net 3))
 (segment (start 27.240662 43.918708) (end 24.437 46.72237) (width 0.75) (layer B.Cu) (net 3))
 (segment (start 24.437 46.72237) (end 24.437 47.709) (width 0.75) (layer B.Cu) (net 3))
 (segment (start 24.437 47.709) (end 24.437 49.475) (width 0.75) (layer B.Cu) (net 3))
 (segment (start 33.340419 36.14) (end 37.378418 40.177999) (width 0.75) (layer B.Cu) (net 3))
 (segment (start 37.378418 40.177999) (end 39.690419 40.177999) (width 0.75) (layer B.Cu) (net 3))
 (segment (start 39.690419 40.177999) (end 39.690419 49.461581) (width 0.75) (layer B.Cu) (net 3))
 (segment (start 39.690419 49.461581) (end 39.677 49.475) (width 0.75) (layer B.Cu) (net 3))
 (segment (start 24.437 47.709) (end 23.710999 46.982999) (width 0.75) (layer B.Cu) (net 3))
 (segment (start 23.710999 46.982999) (end 20.715419 46.982999) (width 0.75) (layer B.Cu) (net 3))
 (segment (start 20.715419 46.982999) (end 19.315419 46.982999) (width 0.75) (layer B.Cu) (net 3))
 (segment (start 41.743619 16.047999) (end 41.974419 16.047999) (width 0.75) (layer B.Cu) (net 3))
 (segment (start 41.974419 16.047999) (end 42.358609 16.432189) (width 0.75) (layer B.Cu) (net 3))
 (segment (start 42.358609 16.432189) (end 42.358609 17.195364) (width 0.75) (layer B.Cu) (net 3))
 (segment (start 42.358609 17.195364) (end 46.556234 21.392989) (width 0.75) (layer B.Cu) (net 3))
 (segment (start 46.556234 21.392989) (end 48.988609 21.392989) (width 0.75) (layer B.Cu) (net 3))
 (segment (start 48.988609 21.392989) (end 49.363619 21.767999) (width 0.75) (layer B.Cu) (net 3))
 (segment (start 49.363619 21.767999) (end 49.363619 23.667999) (width 0.75) (layer B.Cu) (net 3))
 (segment (start 41.743619 16.397999) (end 41.743619 16.047999) (width 0.75) (layer B.Cu) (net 3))
 (segment (start 19.315419 46.982999) (end 15.995419 46.982999) (width 0.75) (layer B.Cu) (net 3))
 (segment (start 15.995419 46.982999) (end 14.330419 45.317999) (width 0.75) (layer B.Cu) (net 3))
 (segment (start 14.392919 45.317999) (end 14.330419 45.317999) (width 0.75) (layer B.Cu) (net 3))
 (segment (start 47.297 49.475) (end 53.28222 49.475) (width 0.75) (layer B.Cu) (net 11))
 (segment (start 53.28222 49.475) (end 54.930419 51.123199) (width 0.75) (layer B.Cu) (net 11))
 (segment (start 47.310419 40.177999) (end 47.310419 49.461581) (width 0.75) (layer B.Cu) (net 11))
 (segment (start 47.310419 49.461581) (end 47.297 49.475) (width 0.75) (layer B.Cu) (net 11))
 (segment (start 33.340419 51.607999) (end 33.340419 46.043199) (width 0.75) (layer B.Cu) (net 9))
 (segment (start 28.260419 31.06) (end 30.38491 28.935509) (width 0.75) (layer B.Cu) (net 5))
 (segment (start 30.38491 28.935509) (end 34.360176 28.935509) (width 0.75) (layer B.Cu) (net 5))
 (segment (start 34.360176 28.935509) (end 35.46491 30.040243) (width 0.75) (layer B.Cu) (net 5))
 (segment (start 35.46491 30.040243) (end 35.46491 31.823531) (width 0.75) (layer B.Cu) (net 5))
 (segment (start 35.46491 31.823531) (end 38.511379 34.87) (width 0.75) (layer B.Cu) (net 5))
 (segment (start 38.511379 34.87) (end 39.46242 34.87) (width 0.75) (layer B.Cu) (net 5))
 (segment (start 39.46242 34.87) (end 39.690419 35.097999) (width 0.75) (layer B.Cu) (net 5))
 (segment (start 23.330419 32.857999) (end 26.46242 32.857999) (width 0.75) (layer B.Cu) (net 5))
 (segment (start 26.46242 32.857999) (end 28.260419 31.06) (width 0.75) (layer B.Cu) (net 5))
 (segment (start 17.190419 30.417999) (end 18.939909 30.417999) (width 0.75) (layer B.Cu) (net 5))
 (segment (start 18.939909 30.417999) (end 21.379909 32.857999) (width 0.75) (layer B.Cu) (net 5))
 (segment (start 21.379909 32.857999) (end 21.893579 32.857999) (width 0.75) (layer B.Cu) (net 5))
 (segment (start 21.893579 32.857999) (end 23.330419 32.857999) (width 0.75) (layer B.Cu) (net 5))
 (segment (start 23.330419 30.317999) (end 25.096419 30.317999) (width 0.75) (layer B.Cu) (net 8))
 (segment (start 25.096419 30.317999) (end 33.340419 22.073999) (width 0.75) (layer B.Cu) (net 8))
 (segment (start 33.340419 22.073999) (end 33.340419 20.9) (width 0.75) (layer B.Cu) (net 8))
 (segment (start 33.340419 31.06) (end 33.340419 32.473492) (width 0.75) (layer B.Cu) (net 6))
 (segment (start 33.340419 32.473492) (end 34.882436 34.015509) (width 0.75) (layer B.Cu) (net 6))
 (segment (start 34.882436 34.015509) (end 35.535554 34.015509) (width 0.75) (layer B.Cu) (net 6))
 (segment (start 28.260419 35.883199) (end 20.115619 35.883199) (width 0.75) (layer B.Cu) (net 6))
 (segment (start 20.115619 35.883199) (end 17.190419 32.957999) (width 0.75) (layer B.Cu) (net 6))
 (segment (start 39.690419 37.637999) (end 39.158044 37.637999) (width 0.75) (layer B.Cu) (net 6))
 (segment (start 39.158044 37.637999) (end 35.535554 34.015509) (width 0.75) (layer B.Cu) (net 6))
 (segment (start 35.535554 34.015509) (end 30.128109 34.015509) (width 0.75) (layer B.Cu) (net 6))
 (segment (start 30.128109 34.015509) (end 29.259908 34.88371) (width 0.75) (layer B.Cu) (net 6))
 (segment (start 29.259908 34.88371) (end 28.260419 35.883199) (width 0.75) (layer B.Cu) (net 6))
 (segment (start 46.823619 23.667999) (end 46.823619 25.567999) (width 0.75) (layer B.Cu) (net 14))
 (segment (start 46.823619 25.567999) (end 48.821 27.56538) (width 0.75) (layer B.Cu) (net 14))
 (segment (start 48.821 27.56538) (end 56.247243 27.56538) (width 0.75) (layer B.Cu) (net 14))
 (segment (start 56.247243 27.56538) (end 57.312521 28.630658) (width 0.75) (layer B.Cu) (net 14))
 (segment (start 57.312521 28.630658) (end 57.312521 35.756345) (width 0.75) (layer B.Cu) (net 14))
 (segment (start 57.312521 35.756345) (end 55.430867 37.637999) (width 0.75) (layer B.Cu) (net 14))
 (segment (start 55.430867 37.637999) (end 49.210419 37.637999) (width 0.75) (layer B.Cu) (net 14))
 (segment (start 49.210419 37.637999) (end 47.310419 37.637999) (width 0.75) (layer B.Cu) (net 14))
 (segment (start 46.823619 23.667999) (end 46.823619 24.200374) (width 0.75) (layer B.Cu) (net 14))
 (segment (start 47.842794 37.637999) (end 47.310419 37.637999) (width 0.75) (layer B.Cu) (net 14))
 (segment (start 47.310419 35.097999) (end 47.310419 37.023299) (width 0.75) (layer B.Cu) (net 14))
 (segment (start 47.310419 37.637999) (end 47.310419 37.023299) (width 0.75) (layer B.Cu) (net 14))
 (segment (start 65.33152 30.546659) (end 56.95206 22.167199) (width 0.75) (layer B.Cu) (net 4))
 (segment (start 56.95206 22.167199) (end 55.205619 22.167199) (width 0.75) (layer B.Cu) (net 4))
 (segment (start 65.060819 41.090199) (end 65.060819 38.108847) (width 0.75) (layer B.Cu) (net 4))
 (segment (start 65.060819 38.108847) (end 62.965928 36.013956) (width 0.75) (layer B.Cu) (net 4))
 (segment (start 62.965928 36.013956) (end 62.965928 32.912251) (width 0.75) (layer B.Cu) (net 4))
 (segment (start 62.965928 32.912251) (end 64.481891 31.396288) (width 0.75) (layer B.Cu) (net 4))
 (segment (start 64.481891 31.396288) (end 65.33152 30.546659) (width 0.75) (layer B.Cu) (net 4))
 (segment (start 46.823619 16.047999) (end 46.823619 16.580374) (width 0.75) (layer B.Cu) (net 4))
 (segment (start 46.823619 16.580374) (end 52.411234 22.167989) (width 0.75) (layer B.Cu) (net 4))
 (segment (start 52.411234 22.167989) (end 55.185209 22.167989) (width 0.75) (layer B.Cu) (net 4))
 (segment (start 44.283619 16.047999) (end 46.823619 16.047999) (width 0.75) (layer B.Cu) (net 4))
 (segment (start 51.221044 13.658199) (end 69.683619 13.658199) (width 0.75) (layer B.Cu) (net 15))
 (segment (start 69.683619 13.658199) (end 78.573619 22.548199) (width 0.75) (layer B.Cu) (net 15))
 (segment (start 49.363619 16.047999) (end 49.363619 15.515624) (width 0.75) (layer B.Cu) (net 15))
 (segment (start 49.363619 15.515624) (end 51.221044 13.658199) (width 0.75) (layer B.Cu) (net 15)))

